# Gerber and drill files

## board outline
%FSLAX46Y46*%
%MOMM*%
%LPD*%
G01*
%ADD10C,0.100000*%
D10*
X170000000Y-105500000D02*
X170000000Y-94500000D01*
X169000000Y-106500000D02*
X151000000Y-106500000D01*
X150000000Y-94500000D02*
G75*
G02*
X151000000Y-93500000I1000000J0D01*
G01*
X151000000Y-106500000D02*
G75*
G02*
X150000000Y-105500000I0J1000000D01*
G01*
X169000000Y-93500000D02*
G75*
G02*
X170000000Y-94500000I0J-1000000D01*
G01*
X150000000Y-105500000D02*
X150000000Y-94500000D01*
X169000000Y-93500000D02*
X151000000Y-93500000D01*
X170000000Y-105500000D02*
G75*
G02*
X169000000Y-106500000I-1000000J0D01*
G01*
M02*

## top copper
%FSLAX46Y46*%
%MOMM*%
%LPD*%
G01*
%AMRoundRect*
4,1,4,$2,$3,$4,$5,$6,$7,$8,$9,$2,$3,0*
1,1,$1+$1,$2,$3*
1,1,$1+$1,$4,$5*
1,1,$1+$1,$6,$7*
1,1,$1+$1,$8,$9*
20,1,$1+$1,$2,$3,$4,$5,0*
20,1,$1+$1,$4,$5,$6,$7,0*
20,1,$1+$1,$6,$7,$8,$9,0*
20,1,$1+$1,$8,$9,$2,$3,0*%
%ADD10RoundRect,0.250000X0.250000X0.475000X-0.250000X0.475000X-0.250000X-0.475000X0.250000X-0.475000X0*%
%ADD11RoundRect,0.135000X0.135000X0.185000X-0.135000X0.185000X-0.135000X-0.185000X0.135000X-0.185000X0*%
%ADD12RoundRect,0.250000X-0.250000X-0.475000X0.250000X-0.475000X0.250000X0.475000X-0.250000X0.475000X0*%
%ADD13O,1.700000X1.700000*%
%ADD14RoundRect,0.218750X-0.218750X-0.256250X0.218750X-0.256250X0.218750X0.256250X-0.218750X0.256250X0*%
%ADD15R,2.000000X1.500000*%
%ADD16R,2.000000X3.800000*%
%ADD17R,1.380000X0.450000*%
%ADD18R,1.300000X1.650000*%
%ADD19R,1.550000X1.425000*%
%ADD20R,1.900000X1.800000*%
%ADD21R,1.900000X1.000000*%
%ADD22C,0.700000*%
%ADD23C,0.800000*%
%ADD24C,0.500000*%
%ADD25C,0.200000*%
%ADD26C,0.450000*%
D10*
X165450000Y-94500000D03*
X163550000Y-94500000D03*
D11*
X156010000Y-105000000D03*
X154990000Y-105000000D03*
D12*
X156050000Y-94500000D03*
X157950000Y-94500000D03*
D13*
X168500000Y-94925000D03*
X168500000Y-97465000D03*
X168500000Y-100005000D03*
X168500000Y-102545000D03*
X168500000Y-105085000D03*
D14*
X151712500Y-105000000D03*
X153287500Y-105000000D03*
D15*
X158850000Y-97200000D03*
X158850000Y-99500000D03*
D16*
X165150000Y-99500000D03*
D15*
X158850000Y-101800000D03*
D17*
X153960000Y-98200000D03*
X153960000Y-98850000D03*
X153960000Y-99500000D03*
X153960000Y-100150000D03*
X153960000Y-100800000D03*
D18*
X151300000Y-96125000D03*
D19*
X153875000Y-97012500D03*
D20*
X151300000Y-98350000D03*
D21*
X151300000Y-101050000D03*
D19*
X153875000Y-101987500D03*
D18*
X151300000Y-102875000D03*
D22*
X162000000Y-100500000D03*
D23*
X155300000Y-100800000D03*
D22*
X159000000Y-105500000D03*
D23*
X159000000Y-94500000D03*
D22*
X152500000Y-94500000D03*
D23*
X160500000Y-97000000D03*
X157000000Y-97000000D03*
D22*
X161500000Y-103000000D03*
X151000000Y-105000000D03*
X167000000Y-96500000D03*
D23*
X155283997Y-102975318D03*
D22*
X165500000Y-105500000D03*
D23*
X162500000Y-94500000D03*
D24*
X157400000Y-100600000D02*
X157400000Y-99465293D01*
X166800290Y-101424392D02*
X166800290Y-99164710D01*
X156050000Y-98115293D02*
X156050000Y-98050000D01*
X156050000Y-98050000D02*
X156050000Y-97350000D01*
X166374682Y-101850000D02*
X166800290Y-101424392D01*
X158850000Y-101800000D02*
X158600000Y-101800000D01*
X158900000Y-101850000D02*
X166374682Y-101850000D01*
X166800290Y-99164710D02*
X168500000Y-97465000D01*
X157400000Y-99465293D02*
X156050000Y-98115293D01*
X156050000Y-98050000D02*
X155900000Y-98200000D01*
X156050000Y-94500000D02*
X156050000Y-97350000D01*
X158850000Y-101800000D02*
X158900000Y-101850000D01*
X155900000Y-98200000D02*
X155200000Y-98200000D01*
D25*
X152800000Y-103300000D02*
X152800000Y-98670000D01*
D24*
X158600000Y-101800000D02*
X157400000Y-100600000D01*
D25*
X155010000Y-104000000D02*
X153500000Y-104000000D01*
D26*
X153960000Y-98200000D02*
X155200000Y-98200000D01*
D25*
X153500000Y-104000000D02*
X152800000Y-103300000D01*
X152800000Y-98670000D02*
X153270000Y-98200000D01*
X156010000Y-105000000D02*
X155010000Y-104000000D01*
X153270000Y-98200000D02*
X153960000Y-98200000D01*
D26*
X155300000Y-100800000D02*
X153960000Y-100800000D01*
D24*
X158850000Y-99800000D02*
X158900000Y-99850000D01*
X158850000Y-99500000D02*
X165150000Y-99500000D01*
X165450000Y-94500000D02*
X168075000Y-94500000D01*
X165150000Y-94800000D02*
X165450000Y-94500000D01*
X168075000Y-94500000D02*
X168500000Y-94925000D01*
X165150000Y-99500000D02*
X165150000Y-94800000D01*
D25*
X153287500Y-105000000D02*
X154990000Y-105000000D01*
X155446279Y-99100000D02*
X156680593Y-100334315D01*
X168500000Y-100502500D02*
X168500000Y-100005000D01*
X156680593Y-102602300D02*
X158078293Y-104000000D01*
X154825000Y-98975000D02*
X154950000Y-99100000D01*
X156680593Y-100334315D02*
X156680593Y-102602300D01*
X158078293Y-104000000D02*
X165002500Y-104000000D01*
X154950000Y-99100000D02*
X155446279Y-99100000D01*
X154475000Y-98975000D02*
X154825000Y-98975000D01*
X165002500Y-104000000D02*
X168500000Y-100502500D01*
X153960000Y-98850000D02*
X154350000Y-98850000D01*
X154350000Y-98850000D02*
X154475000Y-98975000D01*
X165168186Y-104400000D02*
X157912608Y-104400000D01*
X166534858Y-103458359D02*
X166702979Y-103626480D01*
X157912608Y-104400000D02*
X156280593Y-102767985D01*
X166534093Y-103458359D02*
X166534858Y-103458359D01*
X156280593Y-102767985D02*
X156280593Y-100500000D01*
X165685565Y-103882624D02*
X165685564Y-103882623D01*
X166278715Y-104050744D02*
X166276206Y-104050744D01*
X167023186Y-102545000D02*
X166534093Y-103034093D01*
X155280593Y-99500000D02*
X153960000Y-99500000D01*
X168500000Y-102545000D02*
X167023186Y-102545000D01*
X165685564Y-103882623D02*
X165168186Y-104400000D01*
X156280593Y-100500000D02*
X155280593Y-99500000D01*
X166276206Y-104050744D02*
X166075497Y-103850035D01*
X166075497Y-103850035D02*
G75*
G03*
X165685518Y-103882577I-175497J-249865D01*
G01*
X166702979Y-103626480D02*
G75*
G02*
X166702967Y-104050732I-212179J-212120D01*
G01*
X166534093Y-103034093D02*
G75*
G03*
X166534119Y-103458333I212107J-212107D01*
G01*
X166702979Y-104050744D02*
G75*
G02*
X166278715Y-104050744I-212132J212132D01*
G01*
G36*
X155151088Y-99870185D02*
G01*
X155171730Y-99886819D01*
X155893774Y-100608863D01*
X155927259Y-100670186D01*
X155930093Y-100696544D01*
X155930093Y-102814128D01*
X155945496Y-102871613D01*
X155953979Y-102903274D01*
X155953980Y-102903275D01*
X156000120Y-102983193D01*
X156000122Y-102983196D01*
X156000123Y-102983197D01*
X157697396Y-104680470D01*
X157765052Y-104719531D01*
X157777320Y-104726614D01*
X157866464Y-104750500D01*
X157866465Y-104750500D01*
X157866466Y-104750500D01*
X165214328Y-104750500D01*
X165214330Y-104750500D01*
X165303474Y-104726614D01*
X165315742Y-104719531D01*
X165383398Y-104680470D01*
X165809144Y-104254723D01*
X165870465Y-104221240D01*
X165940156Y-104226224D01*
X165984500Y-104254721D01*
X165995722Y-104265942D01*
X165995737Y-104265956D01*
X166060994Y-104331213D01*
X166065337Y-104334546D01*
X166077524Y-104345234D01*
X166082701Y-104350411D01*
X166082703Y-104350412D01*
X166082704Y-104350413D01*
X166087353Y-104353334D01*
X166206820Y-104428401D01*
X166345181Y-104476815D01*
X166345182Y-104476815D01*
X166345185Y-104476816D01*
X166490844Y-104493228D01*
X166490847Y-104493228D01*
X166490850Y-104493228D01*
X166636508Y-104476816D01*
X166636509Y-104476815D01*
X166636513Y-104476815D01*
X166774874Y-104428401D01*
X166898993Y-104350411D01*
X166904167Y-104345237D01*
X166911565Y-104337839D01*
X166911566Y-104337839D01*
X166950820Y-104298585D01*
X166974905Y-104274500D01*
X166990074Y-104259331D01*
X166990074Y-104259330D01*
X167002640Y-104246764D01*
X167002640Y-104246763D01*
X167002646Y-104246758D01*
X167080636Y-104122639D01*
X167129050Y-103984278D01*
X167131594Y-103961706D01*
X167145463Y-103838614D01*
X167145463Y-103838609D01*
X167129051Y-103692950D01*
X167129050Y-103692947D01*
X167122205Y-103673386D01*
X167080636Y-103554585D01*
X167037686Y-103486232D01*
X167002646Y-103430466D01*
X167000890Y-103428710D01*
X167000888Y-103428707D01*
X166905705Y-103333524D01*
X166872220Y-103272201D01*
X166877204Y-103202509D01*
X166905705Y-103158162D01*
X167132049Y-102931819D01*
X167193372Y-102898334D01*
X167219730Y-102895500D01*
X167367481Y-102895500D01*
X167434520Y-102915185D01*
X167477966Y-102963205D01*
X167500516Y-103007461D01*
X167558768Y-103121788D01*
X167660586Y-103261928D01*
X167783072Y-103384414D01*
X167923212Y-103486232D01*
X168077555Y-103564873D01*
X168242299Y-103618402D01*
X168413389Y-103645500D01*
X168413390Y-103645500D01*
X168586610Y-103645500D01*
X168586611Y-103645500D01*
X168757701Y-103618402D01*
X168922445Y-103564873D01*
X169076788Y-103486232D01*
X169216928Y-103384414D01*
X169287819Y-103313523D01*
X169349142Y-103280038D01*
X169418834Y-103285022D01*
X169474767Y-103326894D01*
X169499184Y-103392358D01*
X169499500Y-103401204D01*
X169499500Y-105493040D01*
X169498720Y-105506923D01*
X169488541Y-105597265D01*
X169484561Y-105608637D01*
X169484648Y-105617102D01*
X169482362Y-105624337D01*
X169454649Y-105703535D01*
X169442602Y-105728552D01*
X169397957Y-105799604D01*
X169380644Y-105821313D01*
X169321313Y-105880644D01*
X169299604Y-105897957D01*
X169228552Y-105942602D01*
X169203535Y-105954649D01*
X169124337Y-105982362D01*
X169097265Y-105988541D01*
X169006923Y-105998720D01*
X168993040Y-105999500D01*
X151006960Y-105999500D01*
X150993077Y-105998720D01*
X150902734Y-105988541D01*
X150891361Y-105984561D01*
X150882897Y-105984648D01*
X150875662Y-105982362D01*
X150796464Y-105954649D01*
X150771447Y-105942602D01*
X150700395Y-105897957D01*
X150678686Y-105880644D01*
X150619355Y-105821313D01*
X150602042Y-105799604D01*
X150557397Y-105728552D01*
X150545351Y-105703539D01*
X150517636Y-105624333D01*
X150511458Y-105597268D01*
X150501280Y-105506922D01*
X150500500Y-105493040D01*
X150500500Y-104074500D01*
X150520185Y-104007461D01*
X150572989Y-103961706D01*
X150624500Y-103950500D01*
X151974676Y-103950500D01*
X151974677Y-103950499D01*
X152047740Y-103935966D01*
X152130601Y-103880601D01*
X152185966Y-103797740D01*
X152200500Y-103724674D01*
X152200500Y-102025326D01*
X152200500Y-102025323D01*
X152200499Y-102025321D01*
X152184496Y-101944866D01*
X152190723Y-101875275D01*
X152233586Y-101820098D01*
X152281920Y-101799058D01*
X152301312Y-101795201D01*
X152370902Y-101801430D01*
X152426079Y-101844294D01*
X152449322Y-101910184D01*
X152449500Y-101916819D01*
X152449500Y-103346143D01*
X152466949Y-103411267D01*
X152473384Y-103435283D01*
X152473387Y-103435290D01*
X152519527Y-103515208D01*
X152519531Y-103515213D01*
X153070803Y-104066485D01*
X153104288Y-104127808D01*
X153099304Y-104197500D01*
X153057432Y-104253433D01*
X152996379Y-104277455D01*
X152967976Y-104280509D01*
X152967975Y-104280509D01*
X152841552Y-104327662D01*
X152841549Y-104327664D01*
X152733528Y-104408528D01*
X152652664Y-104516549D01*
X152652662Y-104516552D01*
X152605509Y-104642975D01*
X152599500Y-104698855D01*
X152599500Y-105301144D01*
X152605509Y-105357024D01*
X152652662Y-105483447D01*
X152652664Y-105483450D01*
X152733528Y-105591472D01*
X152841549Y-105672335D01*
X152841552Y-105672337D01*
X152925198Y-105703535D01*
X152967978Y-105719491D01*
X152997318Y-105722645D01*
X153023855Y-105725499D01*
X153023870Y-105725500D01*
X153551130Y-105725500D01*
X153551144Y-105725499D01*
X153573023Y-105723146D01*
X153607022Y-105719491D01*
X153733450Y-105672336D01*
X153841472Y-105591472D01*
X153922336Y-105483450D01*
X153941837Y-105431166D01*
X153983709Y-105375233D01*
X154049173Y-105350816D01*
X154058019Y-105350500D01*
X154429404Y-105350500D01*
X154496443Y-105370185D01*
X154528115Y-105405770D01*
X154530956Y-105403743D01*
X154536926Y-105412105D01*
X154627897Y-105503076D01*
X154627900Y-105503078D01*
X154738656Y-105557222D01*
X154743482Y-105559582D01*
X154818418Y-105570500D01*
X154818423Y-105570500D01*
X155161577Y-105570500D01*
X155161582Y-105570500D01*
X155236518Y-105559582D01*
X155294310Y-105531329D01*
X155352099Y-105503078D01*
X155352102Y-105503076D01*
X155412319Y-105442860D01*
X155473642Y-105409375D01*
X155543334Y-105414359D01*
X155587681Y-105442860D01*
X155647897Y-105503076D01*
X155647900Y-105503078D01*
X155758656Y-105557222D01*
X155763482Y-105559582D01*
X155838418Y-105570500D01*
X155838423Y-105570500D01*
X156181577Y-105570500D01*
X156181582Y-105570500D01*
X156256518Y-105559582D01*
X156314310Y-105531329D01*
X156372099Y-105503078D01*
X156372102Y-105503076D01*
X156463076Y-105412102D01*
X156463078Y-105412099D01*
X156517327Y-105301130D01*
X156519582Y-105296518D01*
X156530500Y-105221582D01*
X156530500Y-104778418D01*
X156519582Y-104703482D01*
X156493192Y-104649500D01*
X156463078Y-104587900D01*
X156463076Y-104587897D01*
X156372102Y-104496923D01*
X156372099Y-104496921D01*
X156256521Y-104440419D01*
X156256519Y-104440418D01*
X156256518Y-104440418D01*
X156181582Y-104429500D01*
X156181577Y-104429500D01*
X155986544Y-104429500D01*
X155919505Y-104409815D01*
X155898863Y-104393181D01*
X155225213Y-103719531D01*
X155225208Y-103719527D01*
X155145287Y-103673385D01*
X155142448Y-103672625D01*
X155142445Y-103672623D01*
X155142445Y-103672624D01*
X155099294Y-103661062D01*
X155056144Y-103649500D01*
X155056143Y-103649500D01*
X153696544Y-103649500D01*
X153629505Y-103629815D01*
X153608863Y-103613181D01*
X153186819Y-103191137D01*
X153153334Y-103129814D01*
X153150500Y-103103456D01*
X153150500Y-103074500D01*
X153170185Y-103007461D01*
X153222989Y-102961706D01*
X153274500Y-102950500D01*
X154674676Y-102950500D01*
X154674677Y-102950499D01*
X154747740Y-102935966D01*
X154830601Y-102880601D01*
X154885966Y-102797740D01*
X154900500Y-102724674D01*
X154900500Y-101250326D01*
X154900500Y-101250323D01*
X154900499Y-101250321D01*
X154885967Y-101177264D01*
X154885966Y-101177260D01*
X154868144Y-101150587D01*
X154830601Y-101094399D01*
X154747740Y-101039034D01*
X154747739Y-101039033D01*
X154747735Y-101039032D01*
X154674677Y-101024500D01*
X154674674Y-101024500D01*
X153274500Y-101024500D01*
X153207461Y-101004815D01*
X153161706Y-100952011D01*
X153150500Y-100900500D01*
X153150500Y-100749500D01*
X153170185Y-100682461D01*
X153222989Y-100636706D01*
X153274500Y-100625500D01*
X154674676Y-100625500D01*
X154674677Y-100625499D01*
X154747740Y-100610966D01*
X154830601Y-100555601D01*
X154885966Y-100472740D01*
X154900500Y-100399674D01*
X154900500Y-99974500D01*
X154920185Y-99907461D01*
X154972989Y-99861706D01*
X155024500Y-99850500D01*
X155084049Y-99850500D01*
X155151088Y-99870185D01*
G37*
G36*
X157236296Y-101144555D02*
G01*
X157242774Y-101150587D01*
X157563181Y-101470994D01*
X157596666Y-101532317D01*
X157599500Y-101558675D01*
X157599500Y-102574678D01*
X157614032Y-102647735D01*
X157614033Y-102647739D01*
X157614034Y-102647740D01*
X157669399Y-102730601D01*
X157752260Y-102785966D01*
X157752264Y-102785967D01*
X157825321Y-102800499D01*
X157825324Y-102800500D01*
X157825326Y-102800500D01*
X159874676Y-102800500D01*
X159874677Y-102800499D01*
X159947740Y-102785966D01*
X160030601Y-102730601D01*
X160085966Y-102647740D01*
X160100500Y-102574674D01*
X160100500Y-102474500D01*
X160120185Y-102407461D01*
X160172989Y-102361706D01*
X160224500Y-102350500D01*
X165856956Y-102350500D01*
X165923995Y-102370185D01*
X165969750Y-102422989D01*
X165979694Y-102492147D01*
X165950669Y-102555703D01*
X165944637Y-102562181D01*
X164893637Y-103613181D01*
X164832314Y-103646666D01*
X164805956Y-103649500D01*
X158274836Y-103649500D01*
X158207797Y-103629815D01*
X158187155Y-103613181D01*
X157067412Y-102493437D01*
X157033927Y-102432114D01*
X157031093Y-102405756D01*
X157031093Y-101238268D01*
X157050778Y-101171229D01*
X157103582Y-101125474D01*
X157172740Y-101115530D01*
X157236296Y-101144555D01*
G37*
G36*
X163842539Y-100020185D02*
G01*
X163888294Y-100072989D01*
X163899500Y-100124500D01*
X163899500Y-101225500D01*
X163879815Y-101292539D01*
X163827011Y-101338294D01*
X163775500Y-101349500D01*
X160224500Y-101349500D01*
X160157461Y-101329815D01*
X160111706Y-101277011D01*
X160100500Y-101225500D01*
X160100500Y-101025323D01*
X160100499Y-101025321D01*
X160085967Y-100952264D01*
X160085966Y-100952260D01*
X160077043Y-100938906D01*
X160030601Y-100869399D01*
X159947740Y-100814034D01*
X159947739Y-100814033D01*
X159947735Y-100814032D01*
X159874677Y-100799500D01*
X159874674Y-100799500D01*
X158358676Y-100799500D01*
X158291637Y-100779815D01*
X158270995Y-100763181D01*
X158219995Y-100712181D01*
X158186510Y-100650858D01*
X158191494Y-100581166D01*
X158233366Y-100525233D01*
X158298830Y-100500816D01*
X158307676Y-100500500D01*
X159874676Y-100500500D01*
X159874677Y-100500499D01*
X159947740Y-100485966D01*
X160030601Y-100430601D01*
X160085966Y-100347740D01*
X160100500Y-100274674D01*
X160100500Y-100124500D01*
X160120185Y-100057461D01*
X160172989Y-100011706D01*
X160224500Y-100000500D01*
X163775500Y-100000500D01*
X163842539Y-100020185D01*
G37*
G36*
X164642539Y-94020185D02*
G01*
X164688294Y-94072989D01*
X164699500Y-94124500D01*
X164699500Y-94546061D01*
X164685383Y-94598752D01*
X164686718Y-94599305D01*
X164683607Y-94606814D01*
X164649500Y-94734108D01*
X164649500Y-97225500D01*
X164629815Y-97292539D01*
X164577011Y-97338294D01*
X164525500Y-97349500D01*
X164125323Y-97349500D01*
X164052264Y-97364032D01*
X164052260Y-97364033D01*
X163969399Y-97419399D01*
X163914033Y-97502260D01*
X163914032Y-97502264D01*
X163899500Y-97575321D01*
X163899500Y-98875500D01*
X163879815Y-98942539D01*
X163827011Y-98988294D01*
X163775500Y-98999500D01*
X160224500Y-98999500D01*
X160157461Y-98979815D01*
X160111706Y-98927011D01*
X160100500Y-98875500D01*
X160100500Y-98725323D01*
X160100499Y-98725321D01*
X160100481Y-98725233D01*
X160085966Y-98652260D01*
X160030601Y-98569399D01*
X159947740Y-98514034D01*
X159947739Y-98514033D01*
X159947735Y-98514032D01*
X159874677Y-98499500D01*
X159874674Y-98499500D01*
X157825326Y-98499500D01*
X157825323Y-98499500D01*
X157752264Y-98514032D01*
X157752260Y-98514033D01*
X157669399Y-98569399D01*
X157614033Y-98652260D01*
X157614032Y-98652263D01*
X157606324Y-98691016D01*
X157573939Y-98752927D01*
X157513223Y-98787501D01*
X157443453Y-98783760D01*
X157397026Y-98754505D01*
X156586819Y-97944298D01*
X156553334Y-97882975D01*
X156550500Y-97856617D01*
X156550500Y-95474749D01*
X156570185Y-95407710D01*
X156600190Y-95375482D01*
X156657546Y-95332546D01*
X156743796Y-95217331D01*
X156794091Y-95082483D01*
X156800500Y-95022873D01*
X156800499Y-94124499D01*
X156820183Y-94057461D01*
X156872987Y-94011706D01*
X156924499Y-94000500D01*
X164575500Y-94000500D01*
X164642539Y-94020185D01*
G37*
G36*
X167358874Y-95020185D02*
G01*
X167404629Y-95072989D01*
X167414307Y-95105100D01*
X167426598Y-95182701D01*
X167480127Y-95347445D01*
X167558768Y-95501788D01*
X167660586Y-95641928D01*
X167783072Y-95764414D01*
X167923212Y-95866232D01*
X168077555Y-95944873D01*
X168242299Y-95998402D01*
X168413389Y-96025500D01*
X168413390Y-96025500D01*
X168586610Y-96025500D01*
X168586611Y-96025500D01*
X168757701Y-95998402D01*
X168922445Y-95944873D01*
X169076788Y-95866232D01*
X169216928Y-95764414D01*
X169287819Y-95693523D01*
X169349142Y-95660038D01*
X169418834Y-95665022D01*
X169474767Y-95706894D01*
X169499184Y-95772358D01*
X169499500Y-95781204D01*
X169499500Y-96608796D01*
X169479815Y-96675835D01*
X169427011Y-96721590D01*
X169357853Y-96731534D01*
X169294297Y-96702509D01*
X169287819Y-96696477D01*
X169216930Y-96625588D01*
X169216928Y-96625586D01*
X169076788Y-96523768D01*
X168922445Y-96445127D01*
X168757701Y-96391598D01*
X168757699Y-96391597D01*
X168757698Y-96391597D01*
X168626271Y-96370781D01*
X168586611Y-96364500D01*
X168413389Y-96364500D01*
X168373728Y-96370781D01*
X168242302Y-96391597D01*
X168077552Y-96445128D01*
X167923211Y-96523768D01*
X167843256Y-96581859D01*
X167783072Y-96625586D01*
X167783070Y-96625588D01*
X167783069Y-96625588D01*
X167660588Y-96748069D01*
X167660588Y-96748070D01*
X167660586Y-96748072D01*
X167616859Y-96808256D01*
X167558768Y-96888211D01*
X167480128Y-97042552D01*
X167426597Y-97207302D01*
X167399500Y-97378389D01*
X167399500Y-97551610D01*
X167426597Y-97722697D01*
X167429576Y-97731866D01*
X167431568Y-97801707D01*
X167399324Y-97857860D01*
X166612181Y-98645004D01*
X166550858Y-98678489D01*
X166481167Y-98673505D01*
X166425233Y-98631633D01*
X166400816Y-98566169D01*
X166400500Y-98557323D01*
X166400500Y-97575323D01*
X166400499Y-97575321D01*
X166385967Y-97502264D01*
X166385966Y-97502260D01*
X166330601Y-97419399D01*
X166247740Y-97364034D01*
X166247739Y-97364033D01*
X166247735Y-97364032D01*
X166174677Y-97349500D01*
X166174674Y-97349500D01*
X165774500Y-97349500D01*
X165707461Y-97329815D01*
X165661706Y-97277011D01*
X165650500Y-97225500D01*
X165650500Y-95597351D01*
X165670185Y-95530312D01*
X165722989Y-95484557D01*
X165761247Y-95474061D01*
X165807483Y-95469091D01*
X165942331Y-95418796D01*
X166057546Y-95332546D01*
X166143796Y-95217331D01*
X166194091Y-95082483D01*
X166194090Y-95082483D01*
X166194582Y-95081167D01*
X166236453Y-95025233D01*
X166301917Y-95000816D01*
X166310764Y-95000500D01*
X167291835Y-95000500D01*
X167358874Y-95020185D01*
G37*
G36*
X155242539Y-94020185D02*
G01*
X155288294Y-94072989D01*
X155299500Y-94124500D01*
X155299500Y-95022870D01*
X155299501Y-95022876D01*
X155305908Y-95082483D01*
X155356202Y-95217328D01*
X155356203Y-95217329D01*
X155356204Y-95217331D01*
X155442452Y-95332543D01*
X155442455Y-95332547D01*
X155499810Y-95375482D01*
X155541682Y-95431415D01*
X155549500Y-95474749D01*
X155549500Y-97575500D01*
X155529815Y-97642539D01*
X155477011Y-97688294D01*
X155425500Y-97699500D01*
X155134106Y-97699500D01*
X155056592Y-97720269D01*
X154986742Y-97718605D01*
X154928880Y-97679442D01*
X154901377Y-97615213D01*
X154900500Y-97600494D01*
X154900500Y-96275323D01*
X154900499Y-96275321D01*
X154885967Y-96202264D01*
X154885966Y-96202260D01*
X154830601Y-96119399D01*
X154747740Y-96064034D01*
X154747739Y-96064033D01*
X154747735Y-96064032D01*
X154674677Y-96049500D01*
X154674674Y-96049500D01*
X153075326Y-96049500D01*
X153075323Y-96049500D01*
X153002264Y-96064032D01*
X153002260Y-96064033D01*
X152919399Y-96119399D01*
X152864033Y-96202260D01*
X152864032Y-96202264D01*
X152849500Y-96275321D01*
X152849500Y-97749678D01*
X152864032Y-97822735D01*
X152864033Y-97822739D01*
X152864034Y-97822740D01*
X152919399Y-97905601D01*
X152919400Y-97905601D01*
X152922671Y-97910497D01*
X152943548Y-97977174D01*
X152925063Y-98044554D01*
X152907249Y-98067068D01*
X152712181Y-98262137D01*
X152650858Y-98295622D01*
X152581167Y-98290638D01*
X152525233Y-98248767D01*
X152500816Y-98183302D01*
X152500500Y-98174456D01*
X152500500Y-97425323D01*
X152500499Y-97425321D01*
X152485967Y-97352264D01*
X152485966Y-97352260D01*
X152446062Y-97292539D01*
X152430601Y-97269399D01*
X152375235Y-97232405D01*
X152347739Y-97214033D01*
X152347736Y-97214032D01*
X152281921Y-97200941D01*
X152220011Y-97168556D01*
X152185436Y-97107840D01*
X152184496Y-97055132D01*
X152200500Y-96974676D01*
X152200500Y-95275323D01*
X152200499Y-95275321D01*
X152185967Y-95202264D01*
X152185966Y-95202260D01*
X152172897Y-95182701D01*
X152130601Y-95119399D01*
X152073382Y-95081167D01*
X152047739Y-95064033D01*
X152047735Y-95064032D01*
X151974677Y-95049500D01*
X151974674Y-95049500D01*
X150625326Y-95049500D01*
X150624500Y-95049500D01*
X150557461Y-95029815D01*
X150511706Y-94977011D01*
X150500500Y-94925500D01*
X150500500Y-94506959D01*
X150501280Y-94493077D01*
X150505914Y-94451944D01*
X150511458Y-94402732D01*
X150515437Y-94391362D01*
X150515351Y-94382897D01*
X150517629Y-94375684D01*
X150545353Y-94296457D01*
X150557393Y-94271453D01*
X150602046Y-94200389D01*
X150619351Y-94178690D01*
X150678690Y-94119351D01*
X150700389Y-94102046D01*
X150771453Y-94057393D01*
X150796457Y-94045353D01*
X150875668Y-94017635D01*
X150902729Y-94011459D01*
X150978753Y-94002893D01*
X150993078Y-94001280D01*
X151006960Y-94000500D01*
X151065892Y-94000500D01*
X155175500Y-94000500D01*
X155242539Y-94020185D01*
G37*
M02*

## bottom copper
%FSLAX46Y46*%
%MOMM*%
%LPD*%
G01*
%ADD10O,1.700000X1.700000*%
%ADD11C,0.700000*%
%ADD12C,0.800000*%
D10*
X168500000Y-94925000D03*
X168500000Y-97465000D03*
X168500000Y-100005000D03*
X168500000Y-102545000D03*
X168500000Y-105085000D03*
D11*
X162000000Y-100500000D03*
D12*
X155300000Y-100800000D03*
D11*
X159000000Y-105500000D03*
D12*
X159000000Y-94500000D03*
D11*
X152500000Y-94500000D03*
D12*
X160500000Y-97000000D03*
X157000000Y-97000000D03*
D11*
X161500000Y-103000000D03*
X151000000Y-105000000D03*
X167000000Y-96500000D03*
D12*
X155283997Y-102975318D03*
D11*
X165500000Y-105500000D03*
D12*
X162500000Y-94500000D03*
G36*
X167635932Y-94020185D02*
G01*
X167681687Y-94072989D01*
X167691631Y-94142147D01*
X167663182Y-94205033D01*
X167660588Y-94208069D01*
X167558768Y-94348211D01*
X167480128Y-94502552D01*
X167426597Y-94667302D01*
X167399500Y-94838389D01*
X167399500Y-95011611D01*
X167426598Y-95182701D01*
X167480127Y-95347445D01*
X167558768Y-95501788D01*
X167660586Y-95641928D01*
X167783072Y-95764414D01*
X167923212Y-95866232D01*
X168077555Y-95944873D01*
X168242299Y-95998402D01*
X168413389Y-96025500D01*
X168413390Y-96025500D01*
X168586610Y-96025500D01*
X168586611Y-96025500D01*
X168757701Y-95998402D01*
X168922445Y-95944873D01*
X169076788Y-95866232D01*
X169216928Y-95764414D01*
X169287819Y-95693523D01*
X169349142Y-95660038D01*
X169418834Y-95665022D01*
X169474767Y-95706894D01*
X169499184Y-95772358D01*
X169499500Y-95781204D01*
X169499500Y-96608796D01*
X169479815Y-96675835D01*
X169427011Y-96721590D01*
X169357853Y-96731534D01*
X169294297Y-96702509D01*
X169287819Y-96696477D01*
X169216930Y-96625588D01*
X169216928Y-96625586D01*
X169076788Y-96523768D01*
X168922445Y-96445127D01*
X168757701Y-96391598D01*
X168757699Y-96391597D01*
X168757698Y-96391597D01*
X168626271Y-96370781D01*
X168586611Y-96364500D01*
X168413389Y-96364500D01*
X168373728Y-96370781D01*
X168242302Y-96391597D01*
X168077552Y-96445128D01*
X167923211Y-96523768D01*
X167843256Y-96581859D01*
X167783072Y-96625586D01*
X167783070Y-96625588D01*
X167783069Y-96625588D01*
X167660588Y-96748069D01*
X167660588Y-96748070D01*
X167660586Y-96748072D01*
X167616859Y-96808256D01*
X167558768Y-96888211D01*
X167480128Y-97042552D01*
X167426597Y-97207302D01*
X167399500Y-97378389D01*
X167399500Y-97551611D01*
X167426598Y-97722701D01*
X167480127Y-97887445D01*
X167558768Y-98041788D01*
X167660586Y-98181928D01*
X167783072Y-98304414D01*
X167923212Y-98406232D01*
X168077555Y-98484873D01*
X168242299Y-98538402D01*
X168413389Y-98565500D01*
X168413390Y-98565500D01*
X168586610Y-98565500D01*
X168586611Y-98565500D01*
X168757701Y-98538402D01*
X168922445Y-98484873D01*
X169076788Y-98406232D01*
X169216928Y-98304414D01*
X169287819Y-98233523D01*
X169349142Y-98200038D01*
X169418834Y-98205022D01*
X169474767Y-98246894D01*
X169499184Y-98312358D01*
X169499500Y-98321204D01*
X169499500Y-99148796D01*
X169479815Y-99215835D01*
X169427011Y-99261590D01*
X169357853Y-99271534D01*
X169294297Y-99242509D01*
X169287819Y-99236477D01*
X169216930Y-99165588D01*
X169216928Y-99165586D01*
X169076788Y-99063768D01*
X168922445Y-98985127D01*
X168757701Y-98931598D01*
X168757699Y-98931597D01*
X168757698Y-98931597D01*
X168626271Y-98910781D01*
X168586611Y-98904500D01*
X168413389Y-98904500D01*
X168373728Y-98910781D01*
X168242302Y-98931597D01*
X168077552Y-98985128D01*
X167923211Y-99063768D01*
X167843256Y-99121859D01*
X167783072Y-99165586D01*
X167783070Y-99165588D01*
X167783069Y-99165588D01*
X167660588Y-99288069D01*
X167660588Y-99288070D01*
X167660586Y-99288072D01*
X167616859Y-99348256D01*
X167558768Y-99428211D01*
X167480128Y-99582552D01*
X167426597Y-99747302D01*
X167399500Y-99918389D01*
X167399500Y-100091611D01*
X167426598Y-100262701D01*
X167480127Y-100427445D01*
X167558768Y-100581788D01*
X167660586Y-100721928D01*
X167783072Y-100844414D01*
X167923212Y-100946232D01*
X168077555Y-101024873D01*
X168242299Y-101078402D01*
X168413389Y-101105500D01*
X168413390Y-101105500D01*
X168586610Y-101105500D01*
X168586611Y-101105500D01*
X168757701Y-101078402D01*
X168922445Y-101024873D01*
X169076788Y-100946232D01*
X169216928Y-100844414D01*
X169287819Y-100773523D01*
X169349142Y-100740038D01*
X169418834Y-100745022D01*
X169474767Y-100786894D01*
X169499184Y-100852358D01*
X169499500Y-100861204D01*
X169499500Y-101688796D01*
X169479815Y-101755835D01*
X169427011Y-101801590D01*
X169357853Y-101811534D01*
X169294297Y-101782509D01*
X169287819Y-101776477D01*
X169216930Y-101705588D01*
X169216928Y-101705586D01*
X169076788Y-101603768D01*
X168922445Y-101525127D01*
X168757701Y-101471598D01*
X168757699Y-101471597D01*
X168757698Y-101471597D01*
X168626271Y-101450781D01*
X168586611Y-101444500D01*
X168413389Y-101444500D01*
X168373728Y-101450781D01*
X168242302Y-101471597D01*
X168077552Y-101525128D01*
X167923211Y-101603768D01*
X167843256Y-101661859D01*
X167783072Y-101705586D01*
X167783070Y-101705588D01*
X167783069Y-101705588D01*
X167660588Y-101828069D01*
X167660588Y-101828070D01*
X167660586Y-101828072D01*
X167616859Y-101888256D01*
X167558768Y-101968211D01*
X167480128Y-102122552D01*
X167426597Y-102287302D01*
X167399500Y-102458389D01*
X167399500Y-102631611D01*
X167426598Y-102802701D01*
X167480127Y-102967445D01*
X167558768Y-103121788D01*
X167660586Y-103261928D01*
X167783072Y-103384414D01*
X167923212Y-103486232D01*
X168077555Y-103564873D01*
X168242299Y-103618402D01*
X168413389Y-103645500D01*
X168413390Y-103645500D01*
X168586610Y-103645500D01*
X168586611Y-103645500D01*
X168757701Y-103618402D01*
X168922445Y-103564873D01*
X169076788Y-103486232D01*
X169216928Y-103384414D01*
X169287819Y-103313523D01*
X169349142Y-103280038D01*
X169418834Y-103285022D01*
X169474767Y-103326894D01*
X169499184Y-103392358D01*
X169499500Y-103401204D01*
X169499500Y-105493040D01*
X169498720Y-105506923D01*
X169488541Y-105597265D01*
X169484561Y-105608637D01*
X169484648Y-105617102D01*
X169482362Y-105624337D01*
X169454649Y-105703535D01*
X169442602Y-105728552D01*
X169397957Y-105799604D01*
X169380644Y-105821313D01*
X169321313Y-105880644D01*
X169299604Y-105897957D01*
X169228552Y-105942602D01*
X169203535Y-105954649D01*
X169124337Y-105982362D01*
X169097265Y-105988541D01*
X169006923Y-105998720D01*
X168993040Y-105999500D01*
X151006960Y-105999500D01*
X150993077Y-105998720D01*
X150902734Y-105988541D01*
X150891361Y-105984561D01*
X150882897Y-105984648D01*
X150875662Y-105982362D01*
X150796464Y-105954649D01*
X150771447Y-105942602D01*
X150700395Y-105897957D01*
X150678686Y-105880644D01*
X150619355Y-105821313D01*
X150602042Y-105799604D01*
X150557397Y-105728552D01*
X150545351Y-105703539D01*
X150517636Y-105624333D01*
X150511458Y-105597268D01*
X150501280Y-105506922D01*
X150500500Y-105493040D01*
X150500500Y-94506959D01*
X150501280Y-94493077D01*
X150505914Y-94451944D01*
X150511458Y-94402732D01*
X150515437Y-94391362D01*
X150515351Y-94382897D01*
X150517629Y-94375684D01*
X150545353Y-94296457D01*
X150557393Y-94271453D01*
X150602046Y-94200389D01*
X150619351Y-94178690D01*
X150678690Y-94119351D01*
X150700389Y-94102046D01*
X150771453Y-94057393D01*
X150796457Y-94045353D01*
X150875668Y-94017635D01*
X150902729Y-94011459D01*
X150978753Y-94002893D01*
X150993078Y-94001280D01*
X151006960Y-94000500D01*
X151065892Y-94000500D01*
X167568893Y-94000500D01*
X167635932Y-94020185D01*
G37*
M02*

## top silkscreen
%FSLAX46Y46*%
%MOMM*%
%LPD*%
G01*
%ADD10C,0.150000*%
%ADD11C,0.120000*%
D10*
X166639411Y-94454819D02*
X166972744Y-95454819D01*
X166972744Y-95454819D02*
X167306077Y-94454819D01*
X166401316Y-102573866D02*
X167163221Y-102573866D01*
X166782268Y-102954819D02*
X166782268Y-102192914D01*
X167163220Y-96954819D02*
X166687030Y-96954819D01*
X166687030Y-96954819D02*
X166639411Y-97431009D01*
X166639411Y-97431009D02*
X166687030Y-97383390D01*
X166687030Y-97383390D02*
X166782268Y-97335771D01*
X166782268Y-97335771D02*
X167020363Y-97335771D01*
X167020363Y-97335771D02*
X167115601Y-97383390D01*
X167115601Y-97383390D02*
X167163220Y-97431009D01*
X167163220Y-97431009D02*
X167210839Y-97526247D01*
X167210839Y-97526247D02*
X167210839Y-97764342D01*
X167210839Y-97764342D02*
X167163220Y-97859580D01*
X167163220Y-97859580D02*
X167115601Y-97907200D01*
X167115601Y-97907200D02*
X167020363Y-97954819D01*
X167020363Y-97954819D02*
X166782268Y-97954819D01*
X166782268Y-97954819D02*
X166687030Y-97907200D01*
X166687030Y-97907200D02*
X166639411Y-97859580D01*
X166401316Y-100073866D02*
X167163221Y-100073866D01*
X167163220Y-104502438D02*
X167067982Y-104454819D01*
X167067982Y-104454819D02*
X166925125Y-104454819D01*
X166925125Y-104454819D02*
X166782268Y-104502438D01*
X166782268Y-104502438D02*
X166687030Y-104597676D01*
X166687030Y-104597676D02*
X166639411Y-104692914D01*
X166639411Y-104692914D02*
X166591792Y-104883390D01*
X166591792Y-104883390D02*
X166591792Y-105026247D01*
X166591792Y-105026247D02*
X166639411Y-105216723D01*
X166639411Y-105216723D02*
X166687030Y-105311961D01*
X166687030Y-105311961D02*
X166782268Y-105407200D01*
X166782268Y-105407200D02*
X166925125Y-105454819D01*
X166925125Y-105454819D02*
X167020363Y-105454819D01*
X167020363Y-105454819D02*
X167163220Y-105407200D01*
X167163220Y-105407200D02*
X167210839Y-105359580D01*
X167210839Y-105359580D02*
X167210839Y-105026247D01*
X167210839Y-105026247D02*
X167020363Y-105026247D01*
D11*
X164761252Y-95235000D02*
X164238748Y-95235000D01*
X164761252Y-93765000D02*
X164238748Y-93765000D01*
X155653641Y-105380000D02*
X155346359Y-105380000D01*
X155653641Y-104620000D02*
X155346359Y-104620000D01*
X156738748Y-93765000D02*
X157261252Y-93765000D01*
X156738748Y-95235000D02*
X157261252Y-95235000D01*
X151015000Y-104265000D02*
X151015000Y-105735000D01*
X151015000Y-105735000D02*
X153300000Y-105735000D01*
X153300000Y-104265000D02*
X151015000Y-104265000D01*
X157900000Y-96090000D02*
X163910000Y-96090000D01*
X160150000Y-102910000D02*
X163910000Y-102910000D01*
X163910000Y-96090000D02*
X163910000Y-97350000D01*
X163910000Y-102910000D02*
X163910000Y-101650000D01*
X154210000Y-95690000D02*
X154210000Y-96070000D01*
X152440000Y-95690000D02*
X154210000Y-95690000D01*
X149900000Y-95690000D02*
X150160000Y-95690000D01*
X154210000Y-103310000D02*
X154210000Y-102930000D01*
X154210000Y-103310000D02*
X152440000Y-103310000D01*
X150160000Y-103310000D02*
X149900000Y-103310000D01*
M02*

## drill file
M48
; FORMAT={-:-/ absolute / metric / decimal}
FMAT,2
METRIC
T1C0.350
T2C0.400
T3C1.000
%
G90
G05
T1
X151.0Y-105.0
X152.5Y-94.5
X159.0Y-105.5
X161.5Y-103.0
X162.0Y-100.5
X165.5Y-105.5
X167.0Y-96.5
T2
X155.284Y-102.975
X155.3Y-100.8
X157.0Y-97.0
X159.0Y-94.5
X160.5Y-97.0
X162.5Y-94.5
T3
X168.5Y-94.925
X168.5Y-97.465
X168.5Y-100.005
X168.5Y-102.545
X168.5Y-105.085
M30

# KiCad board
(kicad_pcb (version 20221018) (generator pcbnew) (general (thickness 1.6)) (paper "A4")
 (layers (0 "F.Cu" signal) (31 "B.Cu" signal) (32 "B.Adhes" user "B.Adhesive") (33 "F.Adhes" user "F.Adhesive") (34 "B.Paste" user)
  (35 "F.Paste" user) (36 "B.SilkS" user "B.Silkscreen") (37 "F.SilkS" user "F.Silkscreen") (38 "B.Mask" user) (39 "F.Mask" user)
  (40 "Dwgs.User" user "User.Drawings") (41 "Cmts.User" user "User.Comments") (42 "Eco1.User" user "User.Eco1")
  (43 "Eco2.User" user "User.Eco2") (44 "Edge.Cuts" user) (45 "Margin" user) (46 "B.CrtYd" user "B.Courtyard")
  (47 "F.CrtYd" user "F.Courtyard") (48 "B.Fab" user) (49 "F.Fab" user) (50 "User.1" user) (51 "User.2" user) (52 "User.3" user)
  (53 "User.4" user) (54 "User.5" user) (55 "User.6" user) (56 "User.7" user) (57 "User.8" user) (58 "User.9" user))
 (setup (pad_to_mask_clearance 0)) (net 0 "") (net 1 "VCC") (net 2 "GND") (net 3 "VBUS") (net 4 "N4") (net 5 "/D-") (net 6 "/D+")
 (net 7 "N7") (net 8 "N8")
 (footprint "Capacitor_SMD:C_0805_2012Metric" (layer "F.Cu") (at 164.5 94.5 180)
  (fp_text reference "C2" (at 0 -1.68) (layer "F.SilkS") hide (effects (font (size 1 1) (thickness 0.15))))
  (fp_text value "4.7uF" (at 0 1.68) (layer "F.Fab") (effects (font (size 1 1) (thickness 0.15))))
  (fp_line (start -0.261252 -0.735) (end 0.261252 -0.735) (stroke (width 0.12) (type solid)) (layer "F.SilkS"))
  (fp_line (start -0.261252 0.735) (end 0.261252 0.735) (stroke (width 0.12) (type solid)) (layer "F.SilkS"))
  (pad "1" smd roundrect (at -0.95 0 180) (size 1 1.45) (layers "F.Cu" "F.Paste" "F.Mask") (roundrect_rratio 0.25) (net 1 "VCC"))
  (pad "2" smd roundrect (at 0.95 0 180) (size 1 1.45) (layers "F.Cu" "F.Paste" "F.Mask") (roundrect_rratio 0.25) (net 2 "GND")))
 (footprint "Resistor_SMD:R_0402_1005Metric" (layer "F.Cu") (at 155.5 105 180)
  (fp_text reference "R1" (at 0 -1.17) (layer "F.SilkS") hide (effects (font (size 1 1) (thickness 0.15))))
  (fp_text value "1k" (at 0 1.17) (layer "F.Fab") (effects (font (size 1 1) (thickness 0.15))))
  (fp_line (start -0.153641 -0.38) (end 0.153641 -0.38) (stroke (width 0.12) (type solid)) (layer "F.SilkS"))
  (fp_line (start -0.153641 0.38) (end 0.153641 0.38) (stroke (width 0.12) (type solid)) (layer "F.SilkS"))
  (pad "1" smd roundrect (at -0.51 0 180) (size 0.54 0.64) (layers "F.Cu" "F.Paste" "F.Mask") (roundrect_rratio 0.25) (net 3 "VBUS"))
  (pad "2" smd roundrect (at 0.51 0 180) (size 0.54 0.64) (layers "F.Cu" "F.Paste" "F.Mask") (roundrect_rratio 0.25) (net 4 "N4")))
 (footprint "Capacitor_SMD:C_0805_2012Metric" (layer "F.Cu") (at 157 94.5)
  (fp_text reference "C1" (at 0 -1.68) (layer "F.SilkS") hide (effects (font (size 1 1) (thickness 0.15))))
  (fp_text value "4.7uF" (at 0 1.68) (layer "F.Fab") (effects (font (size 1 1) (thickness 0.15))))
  (fp_line (start -0.261252 -0.735) (end 0.261252 -0.735) (stroke (width 0.12) (type solid)) (layer "F.SilkS"))
  (fp_line (start -0.261252 0.735) (end 0.261252 0.735) (stroke (width 0.12) (type solid)) (layer "F.SilkS"))
  (pad "1" smd roundrect (at -0.95 0) (size 1 1.45) (layers "F.Cu" "F.Paste" "F.Mask") (roundrect_rratio 0.25) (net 3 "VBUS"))
  (pad "2" smd roundrect (at 0.95 0) (size 1 1.45) (layers "F.Cu" "F.Paste" "F.Mask") (roundrect_rratio 0.25) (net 2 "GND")))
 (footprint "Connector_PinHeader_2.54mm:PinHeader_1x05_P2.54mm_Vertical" (layer "F.Cu") (at 168.5 94.925)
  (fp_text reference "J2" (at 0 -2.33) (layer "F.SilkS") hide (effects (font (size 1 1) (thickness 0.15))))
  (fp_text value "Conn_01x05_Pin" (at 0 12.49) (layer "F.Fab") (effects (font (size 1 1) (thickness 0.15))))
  (pad "1" thru_hole oval (at 0 0) (size 1.7 1.7) (drill 1) (layers "*.Cu" "*.Mask") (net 1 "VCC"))
  (pad "2" thru_hole oval (at 0 2.54) (size 1.7 1.7) (drill 1) (layers "*.Cu" "*.Mask") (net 3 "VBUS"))
  (pad "3" thru_hole oval (at 0 5.08) (size 1.7 1.7) (drill 1) (layers "*.Cu" "*.Mask") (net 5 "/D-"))
  (pad "4" thru_hole oval (at 0 7.62) (size 1.7 1.7) (drill 1) (layers "*.Cu" "*.Mask") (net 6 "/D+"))
  (pad "5" thru_hole oval (at 0 10.16) (size 1.7 1.7) (drill 1) (layers "*.Cu" "*.Mask") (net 2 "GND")))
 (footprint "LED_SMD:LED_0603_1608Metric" (layer "F.Cu") (at 152.5 105)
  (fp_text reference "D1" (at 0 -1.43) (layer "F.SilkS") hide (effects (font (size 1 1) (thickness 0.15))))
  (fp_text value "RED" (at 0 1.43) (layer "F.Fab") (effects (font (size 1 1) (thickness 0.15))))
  (fp_line (start -1.485 -0.735) (end -1.485 0.735) (stroke (width 0.12) (type solid)) (layer "F.SilkS"))
  (fp_line (start -1.485 0.735) (end 0.8 0.735) (stroke (width 0.12) (type solid)) (layer "F.SilkS"))
  (fp_line (start 0.8 -0.735) (end -1.485 -0.735) (stroke (width 0.12) (type solid)) (layer "F.SilkS"))
  (pad "1" smd roundrect (at -0.7875 0) (size 0.875 0.95) (layers "F.Cu" "F.Paste" "F.Mask") (roundrect_rratio 0.25) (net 2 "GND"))
  (pad "2" smd roundrect (at 0.7875 0) (size 0.875 0.95) (layers "F.Cu" "F.Paste" "F.Mask") (roundrect_rratio 0.25) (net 4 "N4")))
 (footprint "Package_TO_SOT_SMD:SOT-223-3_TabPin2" (layer "F.Cu") (at 162 99.5)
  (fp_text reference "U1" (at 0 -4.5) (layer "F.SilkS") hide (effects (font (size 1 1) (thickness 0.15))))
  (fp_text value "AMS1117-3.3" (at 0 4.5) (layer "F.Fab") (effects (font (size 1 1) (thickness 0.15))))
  (fp_line (start -4.1 -3.41) (end 1.91 -3.41) (stroke (width 0.12) (type solid)) (layer "F.SilkS"))
  (fp_line (start -1.85 3.41) (end 1.91 3.41) (stroke (width 0.12) (type solid)) (layer "F.SilkS"))
  (fp_line (start 1.91 -3.41) (end 1.91 -2.15) (stroke (width 0.12) (type solid)) (layer "F.SilkS"))
  (fp_line (start 1.91 3.41) (end 1.91 2.15) (stroke (width 0.12) (type solid)) (layer "F.SilkS"))
  (pad "1" smd rect (at -3.15 -2.3) (size 2 1.5) (layers "F.Cu" "F.Paste" "F.Mask") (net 2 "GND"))
  (pad "2" smd rect (at -3.15 0) (size 2 1.5) (layers "F.Cu" "F.Paste" "F.Mask") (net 1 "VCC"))
  (pad "2" smd rect (at 3.15 0) (size 2 3.8) (layers "F.Cu" "F.Paste" "F.Mask") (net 1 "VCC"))
  (pad "3" smd rect (at -3.15 2.3) (size 2 1.5) (layers "F.Cu" "F.Paste" "F.Mask") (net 3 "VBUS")))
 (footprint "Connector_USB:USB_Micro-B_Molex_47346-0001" (layer "F.Cu") (at 152.5 99.5 -90)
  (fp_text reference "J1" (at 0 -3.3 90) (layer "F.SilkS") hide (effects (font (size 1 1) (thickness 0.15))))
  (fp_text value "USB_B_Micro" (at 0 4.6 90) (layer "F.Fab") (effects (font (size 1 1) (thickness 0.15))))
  (fp_line (start -3.81 -1.71) (end -3.43 -1.71) (stroke (width 0.12) (type solid)) (layer "F.SilkS"))
  (fp_line (start -3.81 0.06) (end -3.81 -1.71) (stroke (width 0.12) (type solid)) (layer "F.SilkS"))
  (fp_line (start -3.81 2.6) (end -3.81 2.34) (stroke (width 0.12) (type solid)) (layer "F.SilkS"))
  (fp_line (start 3.81 -1.71) (end 3.43 -1.71) (stroke (width 0.12) (type solid)) (layer "F.SilkS"))
  (fp_line (start 3.81 -1.71) (end 3.81 0.06) (stroke (width 0.12) (type solid)) (layer "F.SilkS"))
  (fp_line (start 3.81 2.34) (end 3.81 2.6) (stroke (width 0.12) (type solid)) (layer "F.SilkS"))
  (pad "1" smd rect (at -1.3 -1.46 270) (size 0.45 1.38) (layers "F.Cu" "F.Paste" "F.Mask") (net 3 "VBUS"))
  (pad "2" smd rect (at -0.65 -1.46 270) (size 0.45 1.38) (layers "F.Cu" "F.Paste" "F.Mask") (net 5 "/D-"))
  (pad "3" smd rect (at 0 -1.46 270) (size 0.45 1.38) (layers "F.Cu" "F.Paste" "F.Mask") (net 6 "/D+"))
  (pad "4" smd rect (at 0.65 -1.46 270) (size 0.45 1.38) (layers "F.Cu" "F.Paste" "F.Mask") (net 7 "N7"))
  (pad "5" smd rect (at 1.3 -1.46 270) (size 0.45 1.38) (layers "F.Cu" "F.Paste" "F.Mask") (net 2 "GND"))
  (pad "6" smd rect (at -3.375 1.2 270) (size 1.65 1.3) (layers "F.Cu" "F.Paste" "F.Mask") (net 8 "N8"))
  (pad "6" smd rect (at -2.4875 -1.375 270) (size 1.425 1.55) (layers "F.Cu" "F.Paste" "F.Mask") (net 8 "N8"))
  (pad "6" smd rect (at -1.15 1.2 270) (size 1.8 1.9) (layers "F.Cu" "F.Paste" "F.Mask") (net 8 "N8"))
  (pad "6" smd rect (at 1.55 1.2 270) (size 1 1.9) (layers "F.Cu" "F.Paste" "F.Mask") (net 8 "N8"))
  (pad "6" smd rect (at 2.4875 -1.375 270) (size 1.425 1.55) (layers "F.Cu" "F.Paste" "F.Mask") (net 8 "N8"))
  (pad "6" smd rect (at 3.375 1.2 270) (size 1.65 1.3) (layers "F.Cu" "F.Paste" "F.Mask") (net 8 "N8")))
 (gr_line (start 170 105.5) (end 170 94.5) (stroke (width 0.1) (type default)) (layer "Edge.Cuts"))
 (gr_line (start 169 106.5) (end 151 106.5) (stroke (width 0.1) (type default)) (layer "Edge.Cuts"))
 (gr_arc (start 150 94.5) (mid 150.292893 93.792893) (end 151 93.5) (stroke (width 0.1) (type default)) (layer "Edge.Cuts"))
 (gr_arc (start 151 106.5) (mid 150.292893 106.207107) (end 150 105.5) (stroke (width 0.1) (type default)) (layer "Edge.Cuts"))
 (gr_arc (start 169 93.5) (mid 169.707107 93.792893) (end 170 94.5) (stroke (width 0.1) (type default)) (layer "Edge.Cuts"))
 (gr_line (start 150 105.5) (end 150 94.5) (stroke (width 0.1) (type default)) (layer "Edge.Cuts"))
 (gr_line (start 169 93.5) (end 151 93.5) (stroke (width 0.1) (type default)) (layer "Edge.Cuts"))
 (gr_arc (start 170 105.5) (mid 169.707107 106.207107) (end 169 106.5) (stroke (width 0.1) (type default)) (layer "Edge.Cuts"))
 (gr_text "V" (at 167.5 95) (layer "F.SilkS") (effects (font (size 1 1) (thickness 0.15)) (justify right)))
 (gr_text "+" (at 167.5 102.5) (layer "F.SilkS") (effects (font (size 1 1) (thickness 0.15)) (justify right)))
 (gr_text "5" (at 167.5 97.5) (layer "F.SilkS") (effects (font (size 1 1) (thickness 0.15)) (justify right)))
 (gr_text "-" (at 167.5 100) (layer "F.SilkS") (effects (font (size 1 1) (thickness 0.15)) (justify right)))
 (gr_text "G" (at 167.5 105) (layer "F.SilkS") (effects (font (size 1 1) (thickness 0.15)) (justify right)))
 (segment (start 157.4 100.6) (end 157.4 99.465293) (width 0.5) (layer "F.Cu") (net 3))
 (segment (start 166.80029 101.424392) (end 166.80029 99.16471) (width 0.5) (layer "F.Cu") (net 3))
 (segment (start 156.05 98.115293) (end 156.05 98.05) (width 0.5) (layer "F.Cu") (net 3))
 (segment (start 156.05 98.05) (end 156.05 97.35) (width 0.5) (layer "F.Cu") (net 3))
 (segment (start 166.374682 101.85) (end 166.80029 101.424392) (width 0.5) (layer "F.Cu") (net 3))
 (segment (start 158.85 101.8) (end 158.6 101.8) (width 0.5) (layer "F.Cu") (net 3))
 (segment (start 158.9 101.85) (end 166.374682 101.85) (width 0.5) (layer "F.Cu") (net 3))
 (segment (start 166.80029 99.16471) (end 168.5 97.465) (width 0.5) (layer "F.Cu") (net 3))
 (segment (start 157.4 99.465293) (end 156.05 98.115293) (width 0.5) (layer "F.Cu") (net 3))
 (segment (start 156.05 98.05) (end 155.9 98.2) (width 0.5) (layer "F.Cu") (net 3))
 (segment (start 156.05 94.5) (end 156.05 97.35) (width 0.5) (layer "F.Cu") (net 3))
 (segment (start 158.85 101.8) (end 158.9 101.85) (width 0.5) (layer "F.Cu") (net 3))
 (segment (start 155.9 98.2) (end 155.2 98.2) (width 0.5) (layer "F.Cu") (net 3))
 (segment (start 152.8 103.3) (end 152.8 98.67) (width 0.2) (layer "F.Cu") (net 3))
 (segment (start 158.6 101.8) (end 157.4 100.6) (width 0.5) (layer "F.Cu") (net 3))
 (segment (start 155.01 104) (end 153.5 104) (width 0.2) (layer "F.Cu") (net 3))
 (segment (start 153.96 98.2) (end 155.2 98.2) (width 0.45) (layer "F.Cu") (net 3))
 (segment (start 153.5 104) (end 152.8 103.3) (width 0.2) (layer "F.Cu") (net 3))
 (segment (start 152.8 98.67) (end 153.27 98.2) (width 0.2) (layer "F.Cu") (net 3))
 (segment (start 156.01 105) (end 155.01 104) (width 0.2) (layer "F.Cu") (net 3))
 (segment (start 153.27 98.2) (end 153.96 98.2) (width 0.2) (layer "F.Cu") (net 3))
 (segment (start 155.3 100.8) (end 153.96 100.8) (width 0.45) (layer "F.Cu") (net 2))
 (via (at 162 100.5) (size 0.7) (drill 0.35) (layers "F.Cu" "B.Cu") (free) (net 2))
 (via (at 155.3 100.8) (size 0.8) (drill 0.4) (layers "F.Cu" "B.Cu") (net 2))
 (via (at 159 105.5) (size 0.7) (drill 0.35) (layers "F.Cu" "B.Cu") (free) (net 2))
 (via (at 159 94.5) (size 0.8) (drill 0.4) (layers "F.Cu" "B.Cu") (free) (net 2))
 (via (at 152.5 94.5) (size 0.7) (drill 0.35) (layers "F.Cu" "B.Cu") (free) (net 2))
 (via (at 160.5 97) (size 0.8) (drill 0.4) (layers "F.Cu" "B.Cu") (free) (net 2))
 (via (at 157 97) (size 0.8) (drill 0.4) (layers "F.Cu" "B.Cu") (free) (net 2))
 (via (at 161.5 103) (size 0.7) (drill 0.35) (layers "F.Cu" "B.Cu") (free) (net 2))
 (via (at 151 105) (size 0.7) (drill 0.35) (layers "F.Cu" "B.Cu") (free) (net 2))
 (via (at 167 96.5) (size 0.7) (drill 0.35) (layers "F.Cu" "B.Cu") (free) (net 2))
 (via (at 155.283997 102.975318) (size 0.8) (drill 0.4) (layers "F.Cu" "B.Cu") (free) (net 2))
 (via (at 165.5 105.5) (size 0.7) (drill 0.35) (layers "F.Cu" "B.Cu") (free) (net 2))
 (via (at 162.5 94.5) (size 0.8) (drill 0.4) (layers "F.Cu" "B.Cu") (free) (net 2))
 (segment (start 158.85 99.8) (end 158.9 99.85) (width 0.5) (layer "F.Cu") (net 1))
 (segment (start 158.85 99.5) (end 165.15 99.5) (width 0.5) (layer "F.Cu") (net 1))
 (segment (start 165.45 94.5) (end 168.075 94.5) (width 0.5) (layer "F.Cu") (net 1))
 (segment (start 165.15 94.8) (end 165.45 94.5) (width 0.5) (layer "F.Cu") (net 1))
 (segment (start 168.075 94.5) (end 168.5 94.925) (width 0.5) (layer "F.Cu") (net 1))
 (segment (start 165.15 99.5) (end 165.15 94.8) (width 0.5) (layer "F.Cu") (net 1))
 (segment (start 153.2875 105) (end 154.99 105) (width 0.2) (layer "F.Cu") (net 4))
 (segment (start 155.446279 99.1) (end 156.680593 100.334315) (width 0.2) (layer "F.Cu") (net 5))
 (segment (start 168.5 100.5025) (end 168.5 100.005) (width 0.2) (layer "F.Cu") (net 5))
 (segment (start 156.680593 102.6023) (end 158.078293 104) (width 0.2) (layer "F.Cu") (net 5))
 (segment (start 154.825 98.975) (end 154.95 99.1) (width 0.2) (layer "F.Cu") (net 5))
 (segment (start 156.680593 100.334315) (end 156.680593 102.6023) (width 0.2) (layer "F.Cu") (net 5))
 (segment (start 158.078293 104) (end 165.0025 104) (width 0.2) (layer "F.Cu") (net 5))
 (segment (start 154.95 99.1) (end 155.446279 99.1) (width 0.2) (layer "F.Cu") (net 5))
 (segment (start 154.475 98.975) (end 154.825 98.975) (width 0.2) (layer "F.Cu") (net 5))
 (segment (start 165.0025 104) (end 168.5 100.5025) (width 0.2) (layer "F.Cu") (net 5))
 (segment (start 153.96 98.85) (end 154.35 98.85) (width 0.2) (layer "F.Cu") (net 5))
 (segment (start 154.35 98.85) (end 154.475 98.975) (width 0.2) (layer "F.Cu") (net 5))
 (segment (start 165.168186 104.4) (end 157.912608 104.4) (width 0.2) (layer "F.Cu") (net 6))
 (segment (start 166.534858 103.458359) (end 166.702979 103.62648) (width 0.2) (layer "F.Cu") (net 6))
 (segment (start 157.912608 104.4) (end 156.280593 102.767985) (width 0.2) (layer "F.Cu") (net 6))
 (segment (start 166.534093 103.458359) (end 166.534858 103.458359) (width 0.2) (layer "F.Cu") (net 6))
 (segment (start 156.280593 102.767985) (end 156.280593 100.5) (width 0.2) (layer "F.Cu") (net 6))
 (segment (start 165.685565 103.882624) (end 165.685564 103.882623) (width 0.2) (layer "F.Cu") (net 6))
 (segment (start 166.278715 104.050744) (end 166.276206 104.050744) (width 0.2) (layer "F.Cu") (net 6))
 (segment (start 167.023186 102.545) (end 166.534093 103.034093) (width 0.2) (layer "F.Cu") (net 6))
 (segment (start 155.280593 99.5) (end 153.96 99.5) (width 0.2) (layer "F.Cu") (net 6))
 (segment (start 168.5 102.545) (end 167.023186 102.545) (width 0.2) (layer "F.Cu") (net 6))
 (segment (start 165.685564 103.882623) (end 165.168186 104.4) (width 0.2) (layer "F.Cu") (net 6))
 (segment (start 156.280593 100.5) (end 155.280593 99.5) (width 0.2) (layer "F.Cu") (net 6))
 (segment (start 166.276206 104.050744) (end 166.075497 103.850035) (width 0.2) (layer "F.Cu") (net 6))
 (arc (start 166.075497 103.850035) (mid 165.874159 103.795681) (end 165.685565 103.882624) (width 0.2) (layer "F.Cu") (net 6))
 (arc (start 166.702979 103.62648) (mid 166.790847 103.838612) (end 166.702979 104.050744) (width 0.2) (layer "F.Cu") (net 6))
 (arc (start 166.534093 103.034093) (mid 166.446224 103.246227) (end 166.534093 103.458359) (width 0.2) (layer "F.Cu") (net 6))
 (arc (start 166.702979 104.050744) (mid 166.490847 104.138612) (end 166.278715 104.050744) (width 0.2) (layer "F.Cu") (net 6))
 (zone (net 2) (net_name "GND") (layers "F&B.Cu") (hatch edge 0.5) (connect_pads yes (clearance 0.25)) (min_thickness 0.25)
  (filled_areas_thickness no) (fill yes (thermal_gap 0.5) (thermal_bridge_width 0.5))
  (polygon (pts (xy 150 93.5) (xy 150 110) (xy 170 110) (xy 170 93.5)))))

